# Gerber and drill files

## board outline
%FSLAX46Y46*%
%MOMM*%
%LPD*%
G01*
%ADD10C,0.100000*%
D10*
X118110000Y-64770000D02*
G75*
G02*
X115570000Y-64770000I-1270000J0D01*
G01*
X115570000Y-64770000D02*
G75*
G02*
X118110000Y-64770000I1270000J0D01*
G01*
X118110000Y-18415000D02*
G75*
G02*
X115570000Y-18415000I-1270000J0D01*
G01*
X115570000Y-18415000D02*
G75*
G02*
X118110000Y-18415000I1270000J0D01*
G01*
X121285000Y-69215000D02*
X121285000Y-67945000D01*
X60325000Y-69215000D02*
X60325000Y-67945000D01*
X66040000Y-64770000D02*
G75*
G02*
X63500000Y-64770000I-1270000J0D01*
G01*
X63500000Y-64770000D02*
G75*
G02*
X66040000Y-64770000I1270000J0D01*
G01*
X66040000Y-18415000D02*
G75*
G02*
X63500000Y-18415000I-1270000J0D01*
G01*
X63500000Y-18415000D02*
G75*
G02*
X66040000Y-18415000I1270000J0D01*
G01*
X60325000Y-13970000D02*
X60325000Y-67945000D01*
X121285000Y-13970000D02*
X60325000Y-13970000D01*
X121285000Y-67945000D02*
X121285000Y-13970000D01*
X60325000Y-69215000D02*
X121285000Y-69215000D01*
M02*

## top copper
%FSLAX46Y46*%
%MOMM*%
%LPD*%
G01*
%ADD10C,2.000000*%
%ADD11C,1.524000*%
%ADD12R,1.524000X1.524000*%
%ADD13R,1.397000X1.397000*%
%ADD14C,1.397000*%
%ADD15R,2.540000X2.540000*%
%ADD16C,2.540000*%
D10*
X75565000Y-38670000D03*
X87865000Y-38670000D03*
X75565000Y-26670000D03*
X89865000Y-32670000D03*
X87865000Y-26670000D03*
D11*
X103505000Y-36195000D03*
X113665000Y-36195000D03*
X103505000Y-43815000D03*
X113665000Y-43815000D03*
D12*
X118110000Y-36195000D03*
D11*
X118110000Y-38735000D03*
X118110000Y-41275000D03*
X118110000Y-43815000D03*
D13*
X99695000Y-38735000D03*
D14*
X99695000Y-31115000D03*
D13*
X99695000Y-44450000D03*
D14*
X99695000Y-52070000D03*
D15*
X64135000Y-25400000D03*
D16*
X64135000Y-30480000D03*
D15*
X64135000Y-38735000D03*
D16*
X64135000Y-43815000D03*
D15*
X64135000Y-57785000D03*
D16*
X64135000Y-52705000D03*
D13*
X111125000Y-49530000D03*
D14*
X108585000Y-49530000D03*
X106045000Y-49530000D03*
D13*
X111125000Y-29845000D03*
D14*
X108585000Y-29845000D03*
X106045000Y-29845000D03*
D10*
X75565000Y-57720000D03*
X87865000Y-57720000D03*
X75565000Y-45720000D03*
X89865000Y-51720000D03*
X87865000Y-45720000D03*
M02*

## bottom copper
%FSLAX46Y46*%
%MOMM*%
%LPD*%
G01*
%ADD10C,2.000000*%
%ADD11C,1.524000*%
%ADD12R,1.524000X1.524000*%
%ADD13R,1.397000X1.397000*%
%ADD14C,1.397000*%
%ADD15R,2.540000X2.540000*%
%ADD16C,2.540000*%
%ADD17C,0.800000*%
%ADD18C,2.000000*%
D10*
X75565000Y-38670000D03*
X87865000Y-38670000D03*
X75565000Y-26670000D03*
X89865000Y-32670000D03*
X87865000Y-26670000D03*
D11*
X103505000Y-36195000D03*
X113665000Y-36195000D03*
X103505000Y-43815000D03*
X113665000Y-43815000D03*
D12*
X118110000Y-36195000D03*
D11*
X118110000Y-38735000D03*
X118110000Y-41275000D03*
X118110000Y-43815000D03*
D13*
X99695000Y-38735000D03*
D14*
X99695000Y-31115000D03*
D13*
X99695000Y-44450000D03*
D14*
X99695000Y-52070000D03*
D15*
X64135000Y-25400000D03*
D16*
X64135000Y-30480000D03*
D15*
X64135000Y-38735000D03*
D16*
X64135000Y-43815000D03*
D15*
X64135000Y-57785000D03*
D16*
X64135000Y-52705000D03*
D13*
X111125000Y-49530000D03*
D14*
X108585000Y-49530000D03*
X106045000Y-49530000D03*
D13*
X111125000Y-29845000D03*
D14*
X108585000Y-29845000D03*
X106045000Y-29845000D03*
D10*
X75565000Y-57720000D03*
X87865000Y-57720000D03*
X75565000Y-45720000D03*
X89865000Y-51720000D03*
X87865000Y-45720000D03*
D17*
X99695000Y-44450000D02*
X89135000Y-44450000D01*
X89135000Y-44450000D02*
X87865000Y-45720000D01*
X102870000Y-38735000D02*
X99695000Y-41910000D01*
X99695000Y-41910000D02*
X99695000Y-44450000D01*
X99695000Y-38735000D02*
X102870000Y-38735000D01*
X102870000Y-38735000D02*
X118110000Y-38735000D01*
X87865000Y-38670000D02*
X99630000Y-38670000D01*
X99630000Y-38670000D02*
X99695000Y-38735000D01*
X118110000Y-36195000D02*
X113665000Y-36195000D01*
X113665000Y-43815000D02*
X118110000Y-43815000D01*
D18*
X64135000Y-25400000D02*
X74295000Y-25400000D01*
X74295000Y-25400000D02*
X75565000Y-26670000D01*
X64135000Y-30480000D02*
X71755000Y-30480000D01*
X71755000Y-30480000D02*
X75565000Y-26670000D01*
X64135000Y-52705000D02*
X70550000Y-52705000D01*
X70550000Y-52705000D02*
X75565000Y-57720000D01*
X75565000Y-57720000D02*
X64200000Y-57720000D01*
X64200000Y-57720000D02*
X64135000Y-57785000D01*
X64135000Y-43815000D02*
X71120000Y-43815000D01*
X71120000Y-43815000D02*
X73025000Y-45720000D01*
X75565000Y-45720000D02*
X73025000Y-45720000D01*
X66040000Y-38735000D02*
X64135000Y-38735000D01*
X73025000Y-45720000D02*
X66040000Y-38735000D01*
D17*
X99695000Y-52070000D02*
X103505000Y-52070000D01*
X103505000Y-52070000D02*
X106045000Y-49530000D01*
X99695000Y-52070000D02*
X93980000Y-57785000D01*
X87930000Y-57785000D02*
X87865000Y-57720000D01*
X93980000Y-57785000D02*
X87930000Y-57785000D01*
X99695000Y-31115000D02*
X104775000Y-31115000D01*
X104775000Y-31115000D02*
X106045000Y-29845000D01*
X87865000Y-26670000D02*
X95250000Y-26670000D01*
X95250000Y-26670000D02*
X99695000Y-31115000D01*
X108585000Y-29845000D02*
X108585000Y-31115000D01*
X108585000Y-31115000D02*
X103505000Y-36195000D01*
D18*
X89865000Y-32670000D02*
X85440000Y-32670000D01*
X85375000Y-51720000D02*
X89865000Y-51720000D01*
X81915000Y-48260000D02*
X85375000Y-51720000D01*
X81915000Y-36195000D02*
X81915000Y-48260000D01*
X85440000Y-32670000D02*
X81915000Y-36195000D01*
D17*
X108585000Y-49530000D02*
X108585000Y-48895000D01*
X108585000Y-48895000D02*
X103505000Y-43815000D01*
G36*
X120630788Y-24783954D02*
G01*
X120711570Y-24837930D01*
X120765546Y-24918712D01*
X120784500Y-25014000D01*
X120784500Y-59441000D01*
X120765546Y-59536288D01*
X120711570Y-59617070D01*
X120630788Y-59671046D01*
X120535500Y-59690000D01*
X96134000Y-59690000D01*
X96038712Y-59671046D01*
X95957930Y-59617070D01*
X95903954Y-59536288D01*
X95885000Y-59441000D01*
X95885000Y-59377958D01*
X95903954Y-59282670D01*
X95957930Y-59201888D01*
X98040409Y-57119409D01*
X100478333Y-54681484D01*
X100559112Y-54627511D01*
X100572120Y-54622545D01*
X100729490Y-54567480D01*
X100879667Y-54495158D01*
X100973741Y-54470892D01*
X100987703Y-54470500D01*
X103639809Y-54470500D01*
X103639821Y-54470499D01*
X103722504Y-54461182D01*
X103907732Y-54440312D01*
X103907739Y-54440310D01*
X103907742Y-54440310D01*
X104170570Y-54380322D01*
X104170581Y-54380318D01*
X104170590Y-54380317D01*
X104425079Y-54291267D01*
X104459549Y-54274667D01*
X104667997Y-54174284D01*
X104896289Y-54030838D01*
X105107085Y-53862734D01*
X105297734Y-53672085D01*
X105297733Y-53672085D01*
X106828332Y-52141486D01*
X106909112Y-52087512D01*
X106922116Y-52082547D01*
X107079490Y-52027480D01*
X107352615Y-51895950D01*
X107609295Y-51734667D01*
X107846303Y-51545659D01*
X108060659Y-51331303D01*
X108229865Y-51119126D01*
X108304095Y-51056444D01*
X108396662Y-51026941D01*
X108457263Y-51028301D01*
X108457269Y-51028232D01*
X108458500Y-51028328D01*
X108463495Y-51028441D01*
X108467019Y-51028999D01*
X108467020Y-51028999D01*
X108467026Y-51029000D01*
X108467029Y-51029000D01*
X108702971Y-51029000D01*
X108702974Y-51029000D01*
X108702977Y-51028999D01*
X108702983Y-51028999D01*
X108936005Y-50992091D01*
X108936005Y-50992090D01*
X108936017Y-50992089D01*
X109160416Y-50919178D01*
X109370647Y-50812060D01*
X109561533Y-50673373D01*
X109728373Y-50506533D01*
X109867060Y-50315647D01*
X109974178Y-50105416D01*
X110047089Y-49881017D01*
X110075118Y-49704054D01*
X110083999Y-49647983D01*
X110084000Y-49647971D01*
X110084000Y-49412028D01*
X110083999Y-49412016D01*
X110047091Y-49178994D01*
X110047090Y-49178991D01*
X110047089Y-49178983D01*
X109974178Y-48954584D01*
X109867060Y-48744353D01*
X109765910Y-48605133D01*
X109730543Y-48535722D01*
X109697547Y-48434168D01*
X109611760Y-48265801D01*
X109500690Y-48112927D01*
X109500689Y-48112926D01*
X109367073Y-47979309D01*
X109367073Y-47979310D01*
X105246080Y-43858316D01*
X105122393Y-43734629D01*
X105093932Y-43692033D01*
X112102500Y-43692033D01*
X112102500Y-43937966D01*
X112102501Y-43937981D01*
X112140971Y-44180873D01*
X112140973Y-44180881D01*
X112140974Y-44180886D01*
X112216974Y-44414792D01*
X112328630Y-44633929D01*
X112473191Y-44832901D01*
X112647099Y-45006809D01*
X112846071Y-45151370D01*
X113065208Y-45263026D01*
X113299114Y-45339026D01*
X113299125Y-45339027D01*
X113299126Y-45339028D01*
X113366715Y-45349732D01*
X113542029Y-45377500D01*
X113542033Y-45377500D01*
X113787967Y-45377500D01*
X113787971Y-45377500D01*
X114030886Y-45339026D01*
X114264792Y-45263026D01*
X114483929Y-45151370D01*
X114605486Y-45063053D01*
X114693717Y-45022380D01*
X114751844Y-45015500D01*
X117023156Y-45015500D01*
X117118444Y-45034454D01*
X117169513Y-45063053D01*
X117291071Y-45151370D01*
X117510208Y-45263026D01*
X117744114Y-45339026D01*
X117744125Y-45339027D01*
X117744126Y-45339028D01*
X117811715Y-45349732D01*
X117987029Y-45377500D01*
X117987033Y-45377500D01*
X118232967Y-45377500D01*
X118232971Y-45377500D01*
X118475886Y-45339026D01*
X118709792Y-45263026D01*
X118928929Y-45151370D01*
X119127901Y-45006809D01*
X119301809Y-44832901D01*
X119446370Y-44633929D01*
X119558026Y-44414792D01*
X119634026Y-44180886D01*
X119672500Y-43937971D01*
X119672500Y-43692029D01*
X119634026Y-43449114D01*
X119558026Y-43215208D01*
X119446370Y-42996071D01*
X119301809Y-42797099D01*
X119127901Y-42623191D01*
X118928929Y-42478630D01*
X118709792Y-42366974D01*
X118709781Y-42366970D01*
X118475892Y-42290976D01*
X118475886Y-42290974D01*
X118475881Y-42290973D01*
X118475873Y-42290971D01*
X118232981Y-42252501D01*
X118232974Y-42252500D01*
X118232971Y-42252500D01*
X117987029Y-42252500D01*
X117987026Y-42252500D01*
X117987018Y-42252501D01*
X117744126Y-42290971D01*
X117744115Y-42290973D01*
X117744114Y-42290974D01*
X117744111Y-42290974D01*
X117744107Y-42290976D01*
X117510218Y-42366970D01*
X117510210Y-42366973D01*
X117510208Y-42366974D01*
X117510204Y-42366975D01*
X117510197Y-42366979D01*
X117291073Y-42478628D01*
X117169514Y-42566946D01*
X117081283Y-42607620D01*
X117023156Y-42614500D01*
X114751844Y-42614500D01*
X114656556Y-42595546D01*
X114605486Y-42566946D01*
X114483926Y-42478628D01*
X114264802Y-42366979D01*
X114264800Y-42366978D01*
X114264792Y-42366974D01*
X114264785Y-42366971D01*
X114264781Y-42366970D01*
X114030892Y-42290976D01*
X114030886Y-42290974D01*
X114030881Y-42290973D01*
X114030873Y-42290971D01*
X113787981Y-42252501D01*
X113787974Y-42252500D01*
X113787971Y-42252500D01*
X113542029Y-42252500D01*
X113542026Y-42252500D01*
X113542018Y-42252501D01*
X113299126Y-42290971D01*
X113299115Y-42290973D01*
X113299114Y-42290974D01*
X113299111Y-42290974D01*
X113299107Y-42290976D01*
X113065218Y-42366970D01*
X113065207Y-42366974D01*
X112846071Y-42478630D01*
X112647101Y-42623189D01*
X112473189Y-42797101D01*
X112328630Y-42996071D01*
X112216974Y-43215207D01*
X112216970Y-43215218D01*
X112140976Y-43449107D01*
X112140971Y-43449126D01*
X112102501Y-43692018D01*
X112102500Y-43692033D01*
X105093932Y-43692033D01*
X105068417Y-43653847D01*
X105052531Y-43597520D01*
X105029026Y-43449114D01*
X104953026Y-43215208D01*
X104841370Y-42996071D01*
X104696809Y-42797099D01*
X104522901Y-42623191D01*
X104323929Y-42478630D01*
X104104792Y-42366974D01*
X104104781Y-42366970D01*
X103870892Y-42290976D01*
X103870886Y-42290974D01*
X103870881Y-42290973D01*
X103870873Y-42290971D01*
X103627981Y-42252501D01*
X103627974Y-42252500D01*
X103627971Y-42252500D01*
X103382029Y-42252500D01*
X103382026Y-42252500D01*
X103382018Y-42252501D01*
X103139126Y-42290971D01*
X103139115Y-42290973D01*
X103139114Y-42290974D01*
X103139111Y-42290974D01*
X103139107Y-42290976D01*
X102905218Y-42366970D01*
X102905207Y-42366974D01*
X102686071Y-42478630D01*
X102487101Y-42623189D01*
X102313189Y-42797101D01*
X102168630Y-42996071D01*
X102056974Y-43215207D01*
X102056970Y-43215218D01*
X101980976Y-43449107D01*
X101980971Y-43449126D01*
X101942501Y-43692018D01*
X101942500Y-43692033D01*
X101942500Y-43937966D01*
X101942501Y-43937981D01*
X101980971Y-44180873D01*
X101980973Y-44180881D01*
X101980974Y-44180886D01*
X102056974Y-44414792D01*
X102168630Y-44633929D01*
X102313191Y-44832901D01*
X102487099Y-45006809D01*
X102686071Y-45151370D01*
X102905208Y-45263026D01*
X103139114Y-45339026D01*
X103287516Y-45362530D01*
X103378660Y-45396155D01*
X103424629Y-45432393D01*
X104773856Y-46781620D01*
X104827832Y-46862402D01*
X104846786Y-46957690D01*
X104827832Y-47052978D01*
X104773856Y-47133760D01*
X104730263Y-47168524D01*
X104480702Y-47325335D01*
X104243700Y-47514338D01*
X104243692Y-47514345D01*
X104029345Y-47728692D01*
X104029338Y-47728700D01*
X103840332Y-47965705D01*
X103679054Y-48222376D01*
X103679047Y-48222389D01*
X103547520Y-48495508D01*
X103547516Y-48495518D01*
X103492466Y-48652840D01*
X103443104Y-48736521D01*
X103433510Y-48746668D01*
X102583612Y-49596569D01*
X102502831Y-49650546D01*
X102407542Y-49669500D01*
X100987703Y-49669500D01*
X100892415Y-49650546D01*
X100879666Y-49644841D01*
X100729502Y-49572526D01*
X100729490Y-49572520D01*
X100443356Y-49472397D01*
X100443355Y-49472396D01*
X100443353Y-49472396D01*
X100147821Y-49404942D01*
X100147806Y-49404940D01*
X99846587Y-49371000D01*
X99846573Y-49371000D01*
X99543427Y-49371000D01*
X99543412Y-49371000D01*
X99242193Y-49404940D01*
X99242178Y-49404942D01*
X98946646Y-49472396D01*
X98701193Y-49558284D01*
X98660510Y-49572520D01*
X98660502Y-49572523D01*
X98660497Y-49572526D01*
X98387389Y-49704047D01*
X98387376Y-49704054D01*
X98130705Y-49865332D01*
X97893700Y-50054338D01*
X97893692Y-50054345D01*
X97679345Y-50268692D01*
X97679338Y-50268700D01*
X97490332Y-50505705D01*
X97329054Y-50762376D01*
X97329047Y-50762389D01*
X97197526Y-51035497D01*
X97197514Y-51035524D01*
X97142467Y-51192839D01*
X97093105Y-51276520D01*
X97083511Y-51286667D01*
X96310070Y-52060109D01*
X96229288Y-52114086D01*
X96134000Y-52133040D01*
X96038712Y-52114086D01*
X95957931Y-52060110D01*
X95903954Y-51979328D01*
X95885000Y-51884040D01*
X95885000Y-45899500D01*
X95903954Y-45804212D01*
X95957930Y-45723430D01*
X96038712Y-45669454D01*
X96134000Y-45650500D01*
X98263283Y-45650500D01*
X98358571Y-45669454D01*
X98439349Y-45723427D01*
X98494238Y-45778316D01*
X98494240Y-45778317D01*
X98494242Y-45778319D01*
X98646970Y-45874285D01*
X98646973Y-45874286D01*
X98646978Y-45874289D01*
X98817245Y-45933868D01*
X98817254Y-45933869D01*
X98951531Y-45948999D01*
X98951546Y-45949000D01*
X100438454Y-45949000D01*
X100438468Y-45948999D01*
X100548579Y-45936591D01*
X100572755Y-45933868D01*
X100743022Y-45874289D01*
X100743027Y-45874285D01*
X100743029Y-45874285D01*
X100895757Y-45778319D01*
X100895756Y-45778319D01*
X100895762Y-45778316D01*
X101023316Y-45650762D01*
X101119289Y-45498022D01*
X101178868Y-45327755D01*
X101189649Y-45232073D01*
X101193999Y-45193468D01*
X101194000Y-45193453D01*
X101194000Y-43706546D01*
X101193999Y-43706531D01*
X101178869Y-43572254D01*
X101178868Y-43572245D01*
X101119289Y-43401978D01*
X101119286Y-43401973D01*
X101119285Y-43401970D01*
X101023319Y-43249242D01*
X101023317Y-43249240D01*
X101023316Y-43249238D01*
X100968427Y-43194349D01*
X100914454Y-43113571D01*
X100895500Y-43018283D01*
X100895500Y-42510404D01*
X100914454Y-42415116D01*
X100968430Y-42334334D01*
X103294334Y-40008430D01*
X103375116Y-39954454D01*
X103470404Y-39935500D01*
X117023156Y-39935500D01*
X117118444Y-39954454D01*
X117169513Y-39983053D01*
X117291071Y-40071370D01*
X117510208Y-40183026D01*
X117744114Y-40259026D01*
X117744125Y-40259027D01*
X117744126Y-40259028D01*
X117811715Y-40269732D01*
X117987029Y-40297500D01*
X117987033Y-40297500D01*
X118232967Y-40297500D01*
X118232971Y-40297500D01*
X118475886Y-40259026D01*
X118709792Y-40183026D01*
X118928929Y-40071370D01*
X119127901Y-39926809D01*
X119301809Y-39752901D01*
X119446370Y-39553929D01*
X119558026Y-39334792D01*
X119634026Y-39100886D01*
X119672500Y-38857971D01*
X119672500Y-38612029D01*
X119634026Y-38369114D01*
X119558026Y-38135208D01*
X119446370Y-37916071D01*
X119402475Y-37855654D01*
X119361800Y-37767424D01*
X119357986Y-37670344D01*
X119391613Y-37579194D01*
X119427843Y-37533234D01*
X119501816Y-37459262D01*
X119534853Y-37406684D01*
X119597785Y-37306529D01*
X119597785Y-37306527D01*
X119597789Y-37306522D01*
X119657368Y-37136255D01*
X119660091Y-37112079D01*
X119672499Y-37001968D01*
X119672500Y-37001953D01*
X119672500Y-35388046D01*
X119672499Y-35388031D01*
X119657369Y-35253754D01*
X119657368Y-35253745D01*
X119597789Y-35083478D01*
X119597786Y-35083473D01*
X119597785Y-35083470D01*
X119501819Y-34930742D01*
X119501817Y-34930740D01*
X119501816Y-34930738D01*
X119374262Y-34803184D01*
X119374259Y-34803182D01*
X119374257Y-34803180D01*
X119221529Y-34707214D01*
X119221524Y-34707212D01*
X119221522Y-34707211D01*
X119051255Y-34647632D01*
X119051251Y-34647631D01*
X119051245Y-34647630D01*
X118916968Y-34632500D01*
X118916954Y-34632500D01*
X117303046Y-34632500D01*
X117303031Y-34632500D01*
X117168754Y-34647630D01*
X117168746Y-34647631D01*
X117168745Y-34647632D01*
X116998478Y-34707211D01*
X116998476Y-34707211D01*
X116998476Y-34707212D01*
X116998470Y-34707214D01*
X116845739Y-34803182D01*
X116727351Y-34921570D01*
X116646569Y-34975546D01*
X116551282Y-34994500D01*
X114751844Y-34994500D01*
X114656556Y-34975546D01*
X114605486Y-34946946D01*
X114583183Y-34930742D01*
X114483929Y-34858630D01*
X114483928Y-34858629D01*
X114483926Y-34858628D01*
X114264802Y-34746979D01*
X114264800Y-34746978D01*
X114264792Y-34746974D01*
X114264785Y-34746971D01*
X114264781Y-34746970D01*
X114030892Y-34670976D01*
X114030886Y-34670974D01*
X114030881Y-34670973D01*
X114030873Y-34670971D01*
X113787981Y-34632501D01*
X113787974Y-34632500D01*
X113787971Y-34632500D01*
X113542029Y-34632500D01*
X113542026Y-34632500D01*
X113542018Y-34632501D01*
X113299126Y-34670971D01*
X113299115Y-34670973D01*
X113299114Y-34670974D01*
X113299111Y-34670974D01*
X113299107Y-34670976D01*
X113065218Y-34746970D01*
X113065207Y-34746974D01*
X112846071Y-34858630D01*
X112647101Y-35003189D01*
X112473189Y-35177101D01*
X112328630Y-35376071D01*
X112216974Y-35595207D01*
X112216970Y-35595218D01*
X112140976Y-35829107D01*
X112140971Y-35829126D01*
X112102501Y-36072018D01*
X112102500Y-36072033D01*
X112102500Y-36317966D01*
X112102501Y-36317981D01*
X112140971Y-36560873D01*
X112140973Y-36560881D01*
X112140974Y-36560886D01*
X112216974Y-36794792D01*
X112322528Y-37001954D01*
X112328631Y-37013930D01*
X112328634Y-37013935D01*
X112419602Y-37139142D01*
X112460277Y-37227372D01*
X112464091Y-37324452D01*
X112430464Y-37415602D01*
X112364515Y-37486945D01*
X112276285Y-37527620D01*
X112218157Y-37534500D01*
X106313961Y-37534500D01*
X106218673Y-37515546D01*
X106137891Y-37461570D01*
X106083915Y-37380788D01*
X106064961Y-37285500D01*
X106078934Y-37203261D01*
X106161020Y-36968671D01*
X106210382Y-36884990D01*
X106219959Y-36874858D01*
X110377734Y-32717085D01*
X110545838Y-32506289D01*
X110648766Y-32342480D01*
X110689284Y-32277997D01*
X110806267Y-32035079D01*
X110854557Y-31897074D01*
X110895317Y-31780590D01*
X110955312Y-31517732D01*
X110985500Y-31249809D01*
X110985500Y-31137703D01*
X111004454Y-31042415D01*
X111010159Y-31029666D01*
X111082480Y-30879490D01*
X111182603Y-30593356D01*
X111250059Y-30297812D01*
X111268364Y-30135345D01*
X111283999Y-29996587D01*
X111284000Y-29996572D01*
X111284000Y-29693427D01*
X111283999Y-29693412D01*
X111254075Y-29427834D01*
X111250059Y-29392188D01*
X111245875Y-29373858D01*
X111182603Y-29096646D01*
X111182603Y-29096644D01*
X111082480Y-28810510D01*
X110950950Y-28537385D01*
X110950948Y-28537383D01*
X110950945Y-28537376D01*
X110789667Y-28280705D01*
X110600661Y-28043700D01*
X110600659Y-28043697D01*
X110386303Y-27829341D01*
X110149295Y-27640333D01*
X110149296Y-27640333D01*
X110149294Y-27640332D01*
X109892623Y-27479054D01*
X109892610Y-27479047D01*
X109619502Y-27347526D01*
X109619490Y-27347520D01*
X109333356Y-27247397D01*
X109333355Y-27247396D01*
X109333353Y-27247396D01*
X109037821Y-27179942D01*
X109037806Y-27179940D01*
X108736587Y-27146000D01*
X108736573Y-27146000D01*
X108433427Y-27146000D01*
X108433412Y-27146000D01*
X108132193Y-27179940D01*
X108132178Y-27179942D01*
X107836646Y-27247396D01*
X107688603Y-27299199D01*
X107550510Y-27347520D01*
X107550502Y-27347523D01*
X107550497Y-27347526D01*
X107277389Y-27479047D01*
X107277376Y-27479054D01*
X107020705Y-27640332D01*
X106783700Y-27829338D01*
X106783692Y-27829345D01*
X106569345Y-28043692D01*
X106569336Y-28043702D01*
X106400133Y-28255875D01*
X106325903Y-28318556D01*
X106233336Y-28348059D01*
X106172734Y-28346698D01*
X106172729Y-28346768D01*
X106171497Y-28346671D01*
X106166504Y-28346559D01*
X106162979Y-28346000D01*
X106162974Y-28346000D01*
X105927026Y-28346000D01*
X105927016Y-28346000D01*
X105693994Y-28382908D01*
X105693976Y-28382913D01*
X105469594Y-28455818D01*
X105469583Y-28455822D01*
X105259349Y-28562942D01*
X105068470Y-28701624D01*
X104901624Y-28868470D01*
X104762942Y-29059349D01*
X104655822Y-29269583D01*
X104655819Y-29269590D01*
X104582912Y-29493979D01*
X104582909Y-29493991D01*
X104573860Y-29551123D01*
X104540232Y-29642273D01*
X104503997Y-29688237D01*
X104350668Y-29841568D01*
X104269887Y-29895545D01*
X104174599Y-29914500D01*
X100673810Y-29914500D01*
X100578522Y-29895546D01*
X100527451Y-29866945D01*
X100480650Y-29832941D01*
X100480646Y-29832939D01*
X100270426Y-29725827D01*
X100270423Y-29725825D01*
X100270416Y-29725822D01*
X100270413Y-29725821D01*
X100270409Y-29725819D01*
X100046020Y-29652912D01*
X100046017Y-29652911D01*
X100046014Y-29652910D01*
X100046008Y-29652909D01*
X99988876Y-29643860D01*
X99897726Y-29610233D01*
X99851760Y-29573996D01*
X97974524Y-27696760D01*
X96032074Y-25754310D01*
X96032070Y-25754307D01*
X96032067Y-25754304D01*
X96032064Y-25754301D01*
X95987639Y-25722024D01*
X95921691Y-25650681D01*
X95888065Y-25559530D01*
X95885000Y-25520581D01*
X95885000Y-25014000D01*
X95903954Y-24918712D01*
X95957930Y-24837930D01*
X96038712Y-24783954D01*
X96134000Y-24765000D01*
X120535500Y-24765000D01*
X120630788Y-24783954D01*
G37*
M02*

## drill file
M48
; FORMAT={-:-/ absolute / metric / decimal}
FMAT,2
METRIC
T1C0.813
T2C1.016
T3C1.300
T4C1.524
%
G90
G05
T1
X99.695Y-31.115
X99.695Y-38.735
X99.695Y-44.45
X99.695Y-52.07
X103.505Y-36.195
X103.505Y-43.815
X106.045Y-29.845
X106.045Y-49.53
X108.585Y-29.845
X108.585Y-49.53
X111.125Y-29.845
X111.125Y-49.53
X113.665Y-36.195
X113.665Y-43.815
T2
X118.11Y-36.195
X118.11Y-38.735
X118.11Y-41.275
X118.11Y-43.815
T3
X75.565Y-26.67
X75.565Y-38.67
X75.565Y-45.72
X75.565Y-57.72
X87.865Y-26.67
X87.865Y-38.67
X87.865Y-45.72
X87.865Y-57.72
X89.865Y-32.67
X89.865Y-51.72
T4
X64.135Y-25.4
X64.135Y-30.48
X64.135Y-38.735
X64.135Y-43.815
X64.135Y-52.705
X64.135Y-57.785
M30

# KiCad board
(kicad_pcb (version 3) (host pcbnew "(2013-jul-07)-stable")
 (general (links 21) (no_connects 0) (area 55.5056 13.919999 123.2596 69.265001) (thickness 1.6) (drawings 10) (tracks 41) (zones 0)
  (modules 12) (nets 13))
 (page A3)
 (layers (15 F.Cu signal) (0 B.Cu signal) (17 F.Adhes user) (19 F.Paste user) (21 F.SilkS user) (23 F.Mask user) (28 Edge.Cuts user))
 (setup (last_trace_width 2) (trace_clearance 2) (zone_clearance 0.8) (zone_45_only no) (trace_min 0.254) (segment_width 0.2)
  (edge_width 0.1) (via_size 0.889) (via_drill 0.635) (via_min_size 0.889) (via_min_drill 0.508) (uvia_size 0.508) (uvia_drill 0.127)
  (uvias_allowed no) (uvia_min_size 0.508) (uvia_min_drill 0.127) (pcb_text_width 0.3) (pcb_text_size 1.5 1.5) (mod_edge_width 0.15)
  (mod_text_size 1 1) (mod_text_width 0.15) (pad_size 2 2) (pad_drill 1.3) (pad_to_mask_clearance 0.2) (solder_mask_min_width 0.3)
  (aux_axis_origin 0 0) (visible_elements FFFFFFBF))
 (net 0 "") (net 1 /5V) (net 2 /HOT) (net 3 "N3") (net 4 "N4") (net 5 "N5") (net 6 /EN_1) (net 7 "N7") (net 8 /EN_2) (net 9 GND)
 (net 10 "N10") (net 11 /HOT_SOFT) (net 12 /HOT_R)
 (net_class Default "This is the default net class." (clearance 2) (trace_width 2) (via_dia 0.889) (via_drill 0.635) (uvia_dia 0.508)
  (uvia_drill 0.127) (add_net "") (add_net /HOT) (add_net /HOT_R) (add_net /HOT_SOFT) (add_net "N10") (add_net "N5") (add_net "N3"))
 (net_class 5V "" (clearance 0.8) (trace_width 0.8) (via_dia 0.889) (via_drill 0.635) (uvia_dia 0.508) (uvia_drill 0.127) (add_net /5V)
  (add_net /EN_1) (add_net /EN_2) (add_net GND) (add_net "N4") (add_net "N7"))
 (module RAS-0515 (layer F.Cu) (at 75.565 26.67)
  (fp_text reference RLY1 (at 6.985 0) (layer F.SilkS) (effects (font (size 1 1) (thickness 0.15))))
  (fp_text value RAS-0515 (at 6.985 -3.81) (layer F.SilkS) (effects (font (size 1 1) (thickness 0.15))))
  (pad 4 thru_hole circle (at 0 12) (size 2 2) (drill 1.3) (layers *.Cu *.Mask F.SilkS))
  (pad 5 thru_hole circle (at 12.3 12) (size 2 2) (drill 1.3) (layers *.Cu *.Mask F.SilkS) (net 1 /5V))
  (pad 3 thru_hole circle (at 0 0) (size 2 2) (drill 1.3) (layers *.Cu *.Mask F.SilkS) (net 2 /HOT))
  (pad 1 thru_hole circle (at 14.3 6) (size 2 2) (drill 1.3) (layers *.Cu *.Mask F.SilkS) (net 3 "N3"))
  (pad 2 thru_hole circle (at 12.3 0) (size 2 2) (drill 1.3) (layers *.Cu *.Mask F.SilkS) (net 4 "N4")))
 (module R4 (layer F.Cu) (at 108.585 36.195) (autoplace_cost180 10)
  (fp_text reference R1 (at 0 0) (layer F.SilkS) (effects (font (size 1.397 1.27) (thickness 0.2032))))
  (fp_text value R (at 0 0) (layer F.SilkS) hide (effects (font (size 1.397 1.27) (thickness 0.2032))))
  (pad 1 thru_hole circle (at -5.08 0) (size 1.524 1.524) (drill 0.8128) (layers *.Cu *.Mask F.SilkS) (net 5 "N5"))
  (pad 2 thru_hole circle (at 5.08 0) (size 1.524 1.524) (drill 0.8128) (layers *.Cu *.Mask F.SilkS) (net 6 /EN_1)))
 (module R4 (layer F.Cu) (at 108.585 43.815) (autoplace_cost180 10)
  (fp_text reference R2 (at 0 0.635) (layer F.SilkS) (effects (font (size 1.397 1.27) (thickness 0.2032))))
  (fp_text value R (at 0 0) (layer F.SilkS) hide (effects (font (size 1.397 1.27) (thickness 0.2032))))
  (pad 1 thru_hole circle (at -5.08 0) (size 1.524 1.524) (drill 0.8128) (layers *.Cu *.Mask F.SilkS) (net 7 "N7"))
  (pad 2 thru_hole circle (at 5.08 0) (size 1.524 1.524) (drill 0.8128) (layers *.Cu *.Mask F.SilkS) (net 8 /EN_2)))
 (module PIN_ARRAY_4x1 (layer F.Cu) (at 118.11 40.005 270)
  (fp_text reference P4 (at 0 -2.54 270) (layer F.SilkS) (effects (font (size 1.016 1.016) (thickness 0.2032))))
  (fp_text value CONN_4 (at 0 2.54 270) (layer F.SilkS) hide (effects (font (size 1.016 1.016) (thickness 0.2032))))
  (pad 1 thru_hole rect (at -3.81 0 270) (size 1.524 1.524) (drill 1.016) (layers *.Cu *.Mask F.SilkS) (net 6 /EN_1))
  (pad 2 thru_hole circle (at -1.27 0 270) (size 1.524 1.524) (drill 1.016) (layers *.Cu *.Mask F.SilkS) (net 1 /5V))
  (pad 3 thru_hole circle (at 1.27 0 270) (size 1.524 1.524) (drill 1.016) (layers *.Cu *.Mask F.SilkS) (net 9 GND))
  (pad 4 thru_hole circle (at 3.81 0 270) (size 1.524 1.524) (drill 1.016) (layers *.Cu *.Mask F.SilkS) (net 8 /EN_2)))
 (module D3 (layer F.Cu) (at 99.695 34.925 270)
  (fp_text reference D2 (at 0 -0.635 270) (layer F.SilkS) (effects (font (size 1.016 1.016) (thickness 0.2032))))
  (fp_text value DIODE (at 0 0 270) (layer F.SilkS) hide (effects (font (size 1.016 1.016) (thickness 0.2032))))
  (pad 2 thru_hole rect (at 3.81 0 270) (size 1.397 1.397) (drill 0.8128) (layers *.Cu *.Mask F.SilkS) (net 1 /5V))
  (pad 1 thru_hole circle (at -3.81 0 270) (size 1.397 1.397) (drill 0.8128) (layers *.Cu *.Mask F.SilkS) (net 4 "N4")))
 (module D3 (layer F.Cu) (at 99.695 48.26 90)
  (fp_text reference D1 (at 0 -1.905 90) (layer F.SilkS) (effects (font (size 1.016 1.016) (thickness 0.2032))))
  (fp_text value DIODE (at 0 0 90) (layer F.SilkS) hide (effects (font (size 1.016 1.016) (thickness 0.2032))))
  (pad 2 thru_hole rect (at 3.81 0 90) (size 1.397 1.397) (drill 0.8128) (layers *.Cu *.Mask F.SilkS) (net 1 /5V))
  (pad 1 thru_hole circle (at -3.81 0 90) (size 1.397 1.397) (drill 0.8128) (layers *.Cu *.Mask F.SilkS) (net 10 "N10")))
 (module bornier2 (layer F.Cu) (at 64.135 27.94 270)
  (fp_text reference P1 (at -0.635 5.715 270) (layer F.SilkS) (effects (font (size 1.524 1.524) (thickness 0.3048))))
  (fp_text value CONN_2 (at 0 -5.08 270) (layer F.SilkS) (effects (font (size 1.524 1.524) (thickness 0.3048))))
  (pad 1 thru_hole rect (at -2.54 0 270) (size 2.54 2.54) (drill 1.524) (layers *.Cu *.Mask F.SilkS) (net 2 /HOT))
  (pad 2 thru_hole circle (at 2.54 0 270) (size 2.54 2.54) (drill 1.524) (layers *.Cu *.Mask F.SilkS) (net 2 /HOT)))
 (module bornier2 (layer F.Cu) (at 64.135 41.275 270)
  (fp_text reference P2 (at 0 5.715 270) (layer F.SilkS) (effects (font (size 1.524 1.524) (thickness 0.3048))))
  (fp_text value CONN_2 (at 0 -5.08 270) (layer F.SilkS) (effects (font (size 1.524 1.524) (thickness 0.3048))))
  (pad 1 thru_hole rect (at -2.54 0 270) (size 2.54 2.54) (drill 1.524) (layers *.Cu *.Mask F.SilkS) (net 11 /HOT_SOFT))
  (pad 2 thru_hole circle (at 2.54 0 270) (size 2.54 2.54) (drill 1.524) (layers *.Cu *.Mask F.SilkS) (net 11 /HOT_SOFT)))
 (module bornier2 (layer F.Cu) (at 64.135 55.245 90)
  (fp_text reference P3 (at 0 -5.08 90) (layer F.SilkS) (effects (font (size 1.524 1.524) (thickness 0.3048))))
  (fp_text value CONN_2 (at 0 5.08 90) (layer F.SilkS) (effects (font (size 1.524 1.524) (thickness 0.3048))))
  (pad 1 thru_hole rect (at -2.54 0 90) (size 2.54 2.54) (drill 1.524) (layers *.Cu *.Mask F.SilkS) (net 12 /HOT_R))
  (pad 2 thru_hole circle (at 2.54 0 90) (size 2.54 2.54) (drill 1.524) (layers *.Cu *.Mask F.SilkS) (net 12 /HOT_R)))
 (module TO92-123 (layer F.Cu) (at 107.315 50.8 270)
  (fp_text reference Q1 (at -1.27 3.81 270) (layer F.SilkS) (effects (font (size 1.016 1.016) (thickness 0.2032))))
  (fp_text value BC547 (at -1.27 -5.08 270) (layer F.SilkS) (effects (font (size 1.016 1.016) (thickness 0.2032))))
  (pad 3 thru_hole rect (at -1.27 -3.81 270) (size 1.397 1.397) (drill 0.8128) (layers *.Cu *.Mask F.SilkS) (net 9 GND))
  (pad 2 thru_hole circle (at -1.27 -1.27 270) (size 1.397 1.397) (drill 0.8128) (layers *.Cu *.Mask F.SilkS) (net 7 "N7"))
  (pad 1 thru_hole circle (at -1.27 1.27 270) (size 1.397 1.397) (drill 0.8128) (layers *.Cu *.Mask F.SilkS) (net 10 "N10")))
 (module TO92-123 (layer F.Cu) (at 107.315 31.115 270)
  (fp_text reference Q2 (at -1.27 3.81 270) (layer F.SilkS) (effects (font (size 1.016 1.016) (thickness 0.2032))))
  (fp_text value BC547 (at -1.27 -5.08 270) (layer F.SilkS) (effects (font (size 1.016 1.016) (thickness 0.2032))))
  (pad 3 thru_hole rect (at -1.27 -3.81 270) (size 1.397 1.397) (drill 0.8128) (layers *.Cu *.Mask F.SilkS) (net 9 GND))
  (pad 2 thru_hole circle (at -1.27 -1.27 270) (size 1.397 1.397) (drill 0.8128) (layers *.Cu *.Mask F.SilkS) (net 5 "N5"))
  (pad 1 thru_hole circle (at -1.27 1.27 270) (size 1.397 1.397) (drill 0.8128) (layers *.Cu *.Mask F.SilkS) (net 4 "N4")))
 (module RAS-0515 (layer F.Cu) (at 75.565 45.72)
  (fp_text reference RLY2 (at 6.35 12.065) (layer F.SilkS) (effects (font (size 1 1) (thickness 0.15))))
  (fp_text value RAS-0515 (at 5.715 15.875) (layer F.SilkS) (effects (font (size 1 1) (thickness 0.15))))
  (pad 4 thru_hole circle (at 0 12) (size 2 2) (drill 1.3) (layers *.Cu *.Mask F.SilkS) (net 12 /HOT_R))
  (pad 5 thru_hole circle (at 12.3 12) (size 2 2) (drill 1.3) (layers *.Cu *.Mask F.SilkS) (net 10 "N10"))
  (pad 3 thru_hole circle (at 0 0) (size 2 2) (drill 1.3) (layers *.Cu *.Mask F.SilkS) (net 11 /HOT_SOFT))
  (pad 1 thru_hole circle (at 14.3 6) (size 2 2) (drill 1.3) (layers *.Cu *.Mask F.SilkS) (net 3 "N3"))
  (pad 2 thru_hole circle (at 12.3 0) (size 2 2) (drill 1.3) (layers *.Cu *.Mask F.SilkS) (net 1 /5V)))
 (gr_circle (center 116.84 64.77) (end 115.57 64.77) (layer Edge.Cuts) (width 0.1))
 (gr_circle (center 116.84 18.415) (end 115.57 18.415) (layer Edge.Cuts) (width 0.1))
 (gr_line (start 121.285 69.215) (end 121.285 67.945) (angle 90) (layer Edge.Cuts) (width 0.1))
 (gr_line (start 60.325 69.215) (end 60.325 67.945) (angle 90) (layer Edge.Cuts) (width 0.1))
 (gr_circle (center 64.77 64.77) (end 66.04 64.77) (layer Edge.Cuts) (width 0.1))
 (gr_circle (center 64.77 18.415) (end 66.04 18.415) (layer Edge.Cuts) (width 0.1))
 (gr_line (start 60.325 13.97) (end 60.325 67.945) (angle 90) (layer Edge.Cuts) (width 0.1))
 (gr_line (start 121.285 13.97) (end 60.325 13.97) (angle 90) (layer Edge.Cuts) (width 0.1))
 (gr_line (start 121.285 67.945) (end 121.285 13.97) (angle 90) (layer Edge.Cuts) (width 0.1))
 (gr_line (start 60.325 69.215) (end 121.285 69.215) (angle 90) (layer Edge.Cuts) (width 0.1))
 (segment (start 99.695 44.45) (end 89.135 44.45) (width 0.8) (layer B.Cu) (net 1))
 (segment (start 89.135 44.45) (end 87.865 45.72) (width 0.8) (layer B.Cu) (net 1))
 (segment (start 102.87 38.735) (end 99.695 41.91) (width 0.8) (layer B.Cu) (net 1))
 (segment (start 99.695 41.91) (end 99.695 44.45) (width 0.8) (layer B.Cu) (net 1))
 (segment (start 99.695 38.735) (end 102.87 38.735) (width 0.8) (layer B.Cu) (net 1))
 (segment (start 102.87 38.735) (end 118.11 38.735) (width 0.8) (layer B.Cu) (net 1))
 (segment (start 87.865 38.67) (end 99.63 38.67) (width 0.8) (layer B.Cu) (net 1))
 (segment (start 99.63 38.67) (end 99.695 38.735) (width 0.8) (layer B.Cu) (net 1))
 (segment (start 118.11 36.195) (end 113.665 36.195) (width 0.8) (layer B.Cu) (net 6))
 (segment (start 113.665 43.815) (end 118.11 43.815) (width 0.8) (layer B.Cu) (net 8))
 (segment (start 64.135 25.4) (end 74.295 25.4) (width 2) (layer B.Cu) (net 2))
 (segment (start 74.295 25.4) (end 75.565 26.67) (width 2) (layer B.Cu) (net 2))
 (segment (start 64.135 30.48) (end 71.755 30.48) (width 2) (layer B.Cu) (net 2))
 (segment (start 71.755 30.48) (end 75.565 26.67) (width 2) (layer B.Cu) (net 2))
 (segment (start 64.135 52.705) (end 70.55 52.705) (width 2) (layer B.Cu) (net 12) (status 400000))
 (segment (start 70.55 52.705) (end 75.565 57.72) (width 2) (layer B.Cu) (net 12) (status 800000))
 (segment (start 75.565 57.72) (end 64.2 57.72) (width 2) (layer B.Cu) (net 12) (status C00000))
 (segment (start 64.2 57.72) (end 64.135 57.785) (width 2) (layer B.Cu) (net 12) (status C00000))
 (segment (start 64.135 43.815) (end 71.12 43.815) (width 2) (layer B.Cu) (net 11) (status 400000))
 (segment (start 71.12 43.815) (end 73.025 45.72) (width 2) (layer B.Cu) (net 11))
 (segment (start 75.565 45.72) (end 73.025 45.72) (width 2) (layer B.Cu) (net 11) (status 400000))
 (segment (start 66.04 38.735) (end 64.135 38.735) (width 2) (layer B.Cu) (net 11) (status 800000))
 (segment (start 73.025 45.72) (end 66.04 38.735) (width 2) (layer B.Cu) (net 11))
 (segment (start 99.695 52.07) (end 103.505 52.07) (width 0.8) (layer B.Cu) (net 10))
 (segment (start 103.505 52.07) (end 106.045 49.53) (width 0.8) (layer B.Cu) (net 10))
 (segment (start 99.695 52.07) (end 93.98 57.785) (width 0.8) (layer B.Cu) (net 10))
 (segment (start 87.93 57.785) (end 87.865 57.72) (width 0.8) (layer B.Cu) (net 10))
 (segment (start 93.98 57.785) (end 87.93 57.785) (width 0.8) (layer B.Cu) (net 10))
 (segment (start 99.695 31.115) (end 104.775 31.115) (width 0.8) (layer B.Cu) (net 4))
 (segment (start 104.775 31.115) (end 106.045 29.845) (width 0.8) (layer B.Cu) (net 4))
 (segment (start 87.865 26.67) (end 95.25 26.67) (width 0.8) (layer B.Cu) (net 4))
 (segment (start 95.25 26.67) (end 99.695 31.115) (width 0.8) (layer B.Cu) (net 4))
 (segment (start 108.585 29.845) (end 108.585 31.115) (width 0.8) (layer B.Cu) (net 5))
 (segment (start 108.585 31.115) (end 103.505 36.195) (width 0.8) (layer B.Cu) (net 5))
 (segment (start 89.865 32.67) (end 85.44 32.67) (width 2) (layer B.Cu) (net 3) (status 400000))
 (segment (start 85.375 51.72) (end 89.865 51.72) (width 2) (layer B.Cu) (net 3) (status 800000))
 (segment (start 81.915 48.26) (end 85.375 51.72) (width 2) (layer B.Cu) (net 3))
 (segment (start 81.915 36.195) (end 81.915 48.26) (width 2) (layer B.Cu) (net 3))
 (segment (start 85.44 32.67) (end 81.915 36.195) (width 2) (layer B.Cu) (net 3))
 (segment (start 108.585 49.53) (end 108.585 48.895) (width 0.8) (layer B.Cu) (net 7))
 (segment (start 108.585 48.895) (end 103.505 43.815) (width 0.8) (layer B.Cu) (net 7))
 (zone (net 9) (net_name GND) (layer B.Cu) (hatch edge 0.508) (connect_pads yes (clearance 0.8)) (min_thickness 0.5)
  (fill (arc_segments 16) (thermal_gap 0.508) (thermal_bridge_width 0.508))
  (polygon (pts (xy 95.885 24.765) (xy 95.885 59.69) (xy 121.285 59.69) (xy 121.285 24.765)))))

